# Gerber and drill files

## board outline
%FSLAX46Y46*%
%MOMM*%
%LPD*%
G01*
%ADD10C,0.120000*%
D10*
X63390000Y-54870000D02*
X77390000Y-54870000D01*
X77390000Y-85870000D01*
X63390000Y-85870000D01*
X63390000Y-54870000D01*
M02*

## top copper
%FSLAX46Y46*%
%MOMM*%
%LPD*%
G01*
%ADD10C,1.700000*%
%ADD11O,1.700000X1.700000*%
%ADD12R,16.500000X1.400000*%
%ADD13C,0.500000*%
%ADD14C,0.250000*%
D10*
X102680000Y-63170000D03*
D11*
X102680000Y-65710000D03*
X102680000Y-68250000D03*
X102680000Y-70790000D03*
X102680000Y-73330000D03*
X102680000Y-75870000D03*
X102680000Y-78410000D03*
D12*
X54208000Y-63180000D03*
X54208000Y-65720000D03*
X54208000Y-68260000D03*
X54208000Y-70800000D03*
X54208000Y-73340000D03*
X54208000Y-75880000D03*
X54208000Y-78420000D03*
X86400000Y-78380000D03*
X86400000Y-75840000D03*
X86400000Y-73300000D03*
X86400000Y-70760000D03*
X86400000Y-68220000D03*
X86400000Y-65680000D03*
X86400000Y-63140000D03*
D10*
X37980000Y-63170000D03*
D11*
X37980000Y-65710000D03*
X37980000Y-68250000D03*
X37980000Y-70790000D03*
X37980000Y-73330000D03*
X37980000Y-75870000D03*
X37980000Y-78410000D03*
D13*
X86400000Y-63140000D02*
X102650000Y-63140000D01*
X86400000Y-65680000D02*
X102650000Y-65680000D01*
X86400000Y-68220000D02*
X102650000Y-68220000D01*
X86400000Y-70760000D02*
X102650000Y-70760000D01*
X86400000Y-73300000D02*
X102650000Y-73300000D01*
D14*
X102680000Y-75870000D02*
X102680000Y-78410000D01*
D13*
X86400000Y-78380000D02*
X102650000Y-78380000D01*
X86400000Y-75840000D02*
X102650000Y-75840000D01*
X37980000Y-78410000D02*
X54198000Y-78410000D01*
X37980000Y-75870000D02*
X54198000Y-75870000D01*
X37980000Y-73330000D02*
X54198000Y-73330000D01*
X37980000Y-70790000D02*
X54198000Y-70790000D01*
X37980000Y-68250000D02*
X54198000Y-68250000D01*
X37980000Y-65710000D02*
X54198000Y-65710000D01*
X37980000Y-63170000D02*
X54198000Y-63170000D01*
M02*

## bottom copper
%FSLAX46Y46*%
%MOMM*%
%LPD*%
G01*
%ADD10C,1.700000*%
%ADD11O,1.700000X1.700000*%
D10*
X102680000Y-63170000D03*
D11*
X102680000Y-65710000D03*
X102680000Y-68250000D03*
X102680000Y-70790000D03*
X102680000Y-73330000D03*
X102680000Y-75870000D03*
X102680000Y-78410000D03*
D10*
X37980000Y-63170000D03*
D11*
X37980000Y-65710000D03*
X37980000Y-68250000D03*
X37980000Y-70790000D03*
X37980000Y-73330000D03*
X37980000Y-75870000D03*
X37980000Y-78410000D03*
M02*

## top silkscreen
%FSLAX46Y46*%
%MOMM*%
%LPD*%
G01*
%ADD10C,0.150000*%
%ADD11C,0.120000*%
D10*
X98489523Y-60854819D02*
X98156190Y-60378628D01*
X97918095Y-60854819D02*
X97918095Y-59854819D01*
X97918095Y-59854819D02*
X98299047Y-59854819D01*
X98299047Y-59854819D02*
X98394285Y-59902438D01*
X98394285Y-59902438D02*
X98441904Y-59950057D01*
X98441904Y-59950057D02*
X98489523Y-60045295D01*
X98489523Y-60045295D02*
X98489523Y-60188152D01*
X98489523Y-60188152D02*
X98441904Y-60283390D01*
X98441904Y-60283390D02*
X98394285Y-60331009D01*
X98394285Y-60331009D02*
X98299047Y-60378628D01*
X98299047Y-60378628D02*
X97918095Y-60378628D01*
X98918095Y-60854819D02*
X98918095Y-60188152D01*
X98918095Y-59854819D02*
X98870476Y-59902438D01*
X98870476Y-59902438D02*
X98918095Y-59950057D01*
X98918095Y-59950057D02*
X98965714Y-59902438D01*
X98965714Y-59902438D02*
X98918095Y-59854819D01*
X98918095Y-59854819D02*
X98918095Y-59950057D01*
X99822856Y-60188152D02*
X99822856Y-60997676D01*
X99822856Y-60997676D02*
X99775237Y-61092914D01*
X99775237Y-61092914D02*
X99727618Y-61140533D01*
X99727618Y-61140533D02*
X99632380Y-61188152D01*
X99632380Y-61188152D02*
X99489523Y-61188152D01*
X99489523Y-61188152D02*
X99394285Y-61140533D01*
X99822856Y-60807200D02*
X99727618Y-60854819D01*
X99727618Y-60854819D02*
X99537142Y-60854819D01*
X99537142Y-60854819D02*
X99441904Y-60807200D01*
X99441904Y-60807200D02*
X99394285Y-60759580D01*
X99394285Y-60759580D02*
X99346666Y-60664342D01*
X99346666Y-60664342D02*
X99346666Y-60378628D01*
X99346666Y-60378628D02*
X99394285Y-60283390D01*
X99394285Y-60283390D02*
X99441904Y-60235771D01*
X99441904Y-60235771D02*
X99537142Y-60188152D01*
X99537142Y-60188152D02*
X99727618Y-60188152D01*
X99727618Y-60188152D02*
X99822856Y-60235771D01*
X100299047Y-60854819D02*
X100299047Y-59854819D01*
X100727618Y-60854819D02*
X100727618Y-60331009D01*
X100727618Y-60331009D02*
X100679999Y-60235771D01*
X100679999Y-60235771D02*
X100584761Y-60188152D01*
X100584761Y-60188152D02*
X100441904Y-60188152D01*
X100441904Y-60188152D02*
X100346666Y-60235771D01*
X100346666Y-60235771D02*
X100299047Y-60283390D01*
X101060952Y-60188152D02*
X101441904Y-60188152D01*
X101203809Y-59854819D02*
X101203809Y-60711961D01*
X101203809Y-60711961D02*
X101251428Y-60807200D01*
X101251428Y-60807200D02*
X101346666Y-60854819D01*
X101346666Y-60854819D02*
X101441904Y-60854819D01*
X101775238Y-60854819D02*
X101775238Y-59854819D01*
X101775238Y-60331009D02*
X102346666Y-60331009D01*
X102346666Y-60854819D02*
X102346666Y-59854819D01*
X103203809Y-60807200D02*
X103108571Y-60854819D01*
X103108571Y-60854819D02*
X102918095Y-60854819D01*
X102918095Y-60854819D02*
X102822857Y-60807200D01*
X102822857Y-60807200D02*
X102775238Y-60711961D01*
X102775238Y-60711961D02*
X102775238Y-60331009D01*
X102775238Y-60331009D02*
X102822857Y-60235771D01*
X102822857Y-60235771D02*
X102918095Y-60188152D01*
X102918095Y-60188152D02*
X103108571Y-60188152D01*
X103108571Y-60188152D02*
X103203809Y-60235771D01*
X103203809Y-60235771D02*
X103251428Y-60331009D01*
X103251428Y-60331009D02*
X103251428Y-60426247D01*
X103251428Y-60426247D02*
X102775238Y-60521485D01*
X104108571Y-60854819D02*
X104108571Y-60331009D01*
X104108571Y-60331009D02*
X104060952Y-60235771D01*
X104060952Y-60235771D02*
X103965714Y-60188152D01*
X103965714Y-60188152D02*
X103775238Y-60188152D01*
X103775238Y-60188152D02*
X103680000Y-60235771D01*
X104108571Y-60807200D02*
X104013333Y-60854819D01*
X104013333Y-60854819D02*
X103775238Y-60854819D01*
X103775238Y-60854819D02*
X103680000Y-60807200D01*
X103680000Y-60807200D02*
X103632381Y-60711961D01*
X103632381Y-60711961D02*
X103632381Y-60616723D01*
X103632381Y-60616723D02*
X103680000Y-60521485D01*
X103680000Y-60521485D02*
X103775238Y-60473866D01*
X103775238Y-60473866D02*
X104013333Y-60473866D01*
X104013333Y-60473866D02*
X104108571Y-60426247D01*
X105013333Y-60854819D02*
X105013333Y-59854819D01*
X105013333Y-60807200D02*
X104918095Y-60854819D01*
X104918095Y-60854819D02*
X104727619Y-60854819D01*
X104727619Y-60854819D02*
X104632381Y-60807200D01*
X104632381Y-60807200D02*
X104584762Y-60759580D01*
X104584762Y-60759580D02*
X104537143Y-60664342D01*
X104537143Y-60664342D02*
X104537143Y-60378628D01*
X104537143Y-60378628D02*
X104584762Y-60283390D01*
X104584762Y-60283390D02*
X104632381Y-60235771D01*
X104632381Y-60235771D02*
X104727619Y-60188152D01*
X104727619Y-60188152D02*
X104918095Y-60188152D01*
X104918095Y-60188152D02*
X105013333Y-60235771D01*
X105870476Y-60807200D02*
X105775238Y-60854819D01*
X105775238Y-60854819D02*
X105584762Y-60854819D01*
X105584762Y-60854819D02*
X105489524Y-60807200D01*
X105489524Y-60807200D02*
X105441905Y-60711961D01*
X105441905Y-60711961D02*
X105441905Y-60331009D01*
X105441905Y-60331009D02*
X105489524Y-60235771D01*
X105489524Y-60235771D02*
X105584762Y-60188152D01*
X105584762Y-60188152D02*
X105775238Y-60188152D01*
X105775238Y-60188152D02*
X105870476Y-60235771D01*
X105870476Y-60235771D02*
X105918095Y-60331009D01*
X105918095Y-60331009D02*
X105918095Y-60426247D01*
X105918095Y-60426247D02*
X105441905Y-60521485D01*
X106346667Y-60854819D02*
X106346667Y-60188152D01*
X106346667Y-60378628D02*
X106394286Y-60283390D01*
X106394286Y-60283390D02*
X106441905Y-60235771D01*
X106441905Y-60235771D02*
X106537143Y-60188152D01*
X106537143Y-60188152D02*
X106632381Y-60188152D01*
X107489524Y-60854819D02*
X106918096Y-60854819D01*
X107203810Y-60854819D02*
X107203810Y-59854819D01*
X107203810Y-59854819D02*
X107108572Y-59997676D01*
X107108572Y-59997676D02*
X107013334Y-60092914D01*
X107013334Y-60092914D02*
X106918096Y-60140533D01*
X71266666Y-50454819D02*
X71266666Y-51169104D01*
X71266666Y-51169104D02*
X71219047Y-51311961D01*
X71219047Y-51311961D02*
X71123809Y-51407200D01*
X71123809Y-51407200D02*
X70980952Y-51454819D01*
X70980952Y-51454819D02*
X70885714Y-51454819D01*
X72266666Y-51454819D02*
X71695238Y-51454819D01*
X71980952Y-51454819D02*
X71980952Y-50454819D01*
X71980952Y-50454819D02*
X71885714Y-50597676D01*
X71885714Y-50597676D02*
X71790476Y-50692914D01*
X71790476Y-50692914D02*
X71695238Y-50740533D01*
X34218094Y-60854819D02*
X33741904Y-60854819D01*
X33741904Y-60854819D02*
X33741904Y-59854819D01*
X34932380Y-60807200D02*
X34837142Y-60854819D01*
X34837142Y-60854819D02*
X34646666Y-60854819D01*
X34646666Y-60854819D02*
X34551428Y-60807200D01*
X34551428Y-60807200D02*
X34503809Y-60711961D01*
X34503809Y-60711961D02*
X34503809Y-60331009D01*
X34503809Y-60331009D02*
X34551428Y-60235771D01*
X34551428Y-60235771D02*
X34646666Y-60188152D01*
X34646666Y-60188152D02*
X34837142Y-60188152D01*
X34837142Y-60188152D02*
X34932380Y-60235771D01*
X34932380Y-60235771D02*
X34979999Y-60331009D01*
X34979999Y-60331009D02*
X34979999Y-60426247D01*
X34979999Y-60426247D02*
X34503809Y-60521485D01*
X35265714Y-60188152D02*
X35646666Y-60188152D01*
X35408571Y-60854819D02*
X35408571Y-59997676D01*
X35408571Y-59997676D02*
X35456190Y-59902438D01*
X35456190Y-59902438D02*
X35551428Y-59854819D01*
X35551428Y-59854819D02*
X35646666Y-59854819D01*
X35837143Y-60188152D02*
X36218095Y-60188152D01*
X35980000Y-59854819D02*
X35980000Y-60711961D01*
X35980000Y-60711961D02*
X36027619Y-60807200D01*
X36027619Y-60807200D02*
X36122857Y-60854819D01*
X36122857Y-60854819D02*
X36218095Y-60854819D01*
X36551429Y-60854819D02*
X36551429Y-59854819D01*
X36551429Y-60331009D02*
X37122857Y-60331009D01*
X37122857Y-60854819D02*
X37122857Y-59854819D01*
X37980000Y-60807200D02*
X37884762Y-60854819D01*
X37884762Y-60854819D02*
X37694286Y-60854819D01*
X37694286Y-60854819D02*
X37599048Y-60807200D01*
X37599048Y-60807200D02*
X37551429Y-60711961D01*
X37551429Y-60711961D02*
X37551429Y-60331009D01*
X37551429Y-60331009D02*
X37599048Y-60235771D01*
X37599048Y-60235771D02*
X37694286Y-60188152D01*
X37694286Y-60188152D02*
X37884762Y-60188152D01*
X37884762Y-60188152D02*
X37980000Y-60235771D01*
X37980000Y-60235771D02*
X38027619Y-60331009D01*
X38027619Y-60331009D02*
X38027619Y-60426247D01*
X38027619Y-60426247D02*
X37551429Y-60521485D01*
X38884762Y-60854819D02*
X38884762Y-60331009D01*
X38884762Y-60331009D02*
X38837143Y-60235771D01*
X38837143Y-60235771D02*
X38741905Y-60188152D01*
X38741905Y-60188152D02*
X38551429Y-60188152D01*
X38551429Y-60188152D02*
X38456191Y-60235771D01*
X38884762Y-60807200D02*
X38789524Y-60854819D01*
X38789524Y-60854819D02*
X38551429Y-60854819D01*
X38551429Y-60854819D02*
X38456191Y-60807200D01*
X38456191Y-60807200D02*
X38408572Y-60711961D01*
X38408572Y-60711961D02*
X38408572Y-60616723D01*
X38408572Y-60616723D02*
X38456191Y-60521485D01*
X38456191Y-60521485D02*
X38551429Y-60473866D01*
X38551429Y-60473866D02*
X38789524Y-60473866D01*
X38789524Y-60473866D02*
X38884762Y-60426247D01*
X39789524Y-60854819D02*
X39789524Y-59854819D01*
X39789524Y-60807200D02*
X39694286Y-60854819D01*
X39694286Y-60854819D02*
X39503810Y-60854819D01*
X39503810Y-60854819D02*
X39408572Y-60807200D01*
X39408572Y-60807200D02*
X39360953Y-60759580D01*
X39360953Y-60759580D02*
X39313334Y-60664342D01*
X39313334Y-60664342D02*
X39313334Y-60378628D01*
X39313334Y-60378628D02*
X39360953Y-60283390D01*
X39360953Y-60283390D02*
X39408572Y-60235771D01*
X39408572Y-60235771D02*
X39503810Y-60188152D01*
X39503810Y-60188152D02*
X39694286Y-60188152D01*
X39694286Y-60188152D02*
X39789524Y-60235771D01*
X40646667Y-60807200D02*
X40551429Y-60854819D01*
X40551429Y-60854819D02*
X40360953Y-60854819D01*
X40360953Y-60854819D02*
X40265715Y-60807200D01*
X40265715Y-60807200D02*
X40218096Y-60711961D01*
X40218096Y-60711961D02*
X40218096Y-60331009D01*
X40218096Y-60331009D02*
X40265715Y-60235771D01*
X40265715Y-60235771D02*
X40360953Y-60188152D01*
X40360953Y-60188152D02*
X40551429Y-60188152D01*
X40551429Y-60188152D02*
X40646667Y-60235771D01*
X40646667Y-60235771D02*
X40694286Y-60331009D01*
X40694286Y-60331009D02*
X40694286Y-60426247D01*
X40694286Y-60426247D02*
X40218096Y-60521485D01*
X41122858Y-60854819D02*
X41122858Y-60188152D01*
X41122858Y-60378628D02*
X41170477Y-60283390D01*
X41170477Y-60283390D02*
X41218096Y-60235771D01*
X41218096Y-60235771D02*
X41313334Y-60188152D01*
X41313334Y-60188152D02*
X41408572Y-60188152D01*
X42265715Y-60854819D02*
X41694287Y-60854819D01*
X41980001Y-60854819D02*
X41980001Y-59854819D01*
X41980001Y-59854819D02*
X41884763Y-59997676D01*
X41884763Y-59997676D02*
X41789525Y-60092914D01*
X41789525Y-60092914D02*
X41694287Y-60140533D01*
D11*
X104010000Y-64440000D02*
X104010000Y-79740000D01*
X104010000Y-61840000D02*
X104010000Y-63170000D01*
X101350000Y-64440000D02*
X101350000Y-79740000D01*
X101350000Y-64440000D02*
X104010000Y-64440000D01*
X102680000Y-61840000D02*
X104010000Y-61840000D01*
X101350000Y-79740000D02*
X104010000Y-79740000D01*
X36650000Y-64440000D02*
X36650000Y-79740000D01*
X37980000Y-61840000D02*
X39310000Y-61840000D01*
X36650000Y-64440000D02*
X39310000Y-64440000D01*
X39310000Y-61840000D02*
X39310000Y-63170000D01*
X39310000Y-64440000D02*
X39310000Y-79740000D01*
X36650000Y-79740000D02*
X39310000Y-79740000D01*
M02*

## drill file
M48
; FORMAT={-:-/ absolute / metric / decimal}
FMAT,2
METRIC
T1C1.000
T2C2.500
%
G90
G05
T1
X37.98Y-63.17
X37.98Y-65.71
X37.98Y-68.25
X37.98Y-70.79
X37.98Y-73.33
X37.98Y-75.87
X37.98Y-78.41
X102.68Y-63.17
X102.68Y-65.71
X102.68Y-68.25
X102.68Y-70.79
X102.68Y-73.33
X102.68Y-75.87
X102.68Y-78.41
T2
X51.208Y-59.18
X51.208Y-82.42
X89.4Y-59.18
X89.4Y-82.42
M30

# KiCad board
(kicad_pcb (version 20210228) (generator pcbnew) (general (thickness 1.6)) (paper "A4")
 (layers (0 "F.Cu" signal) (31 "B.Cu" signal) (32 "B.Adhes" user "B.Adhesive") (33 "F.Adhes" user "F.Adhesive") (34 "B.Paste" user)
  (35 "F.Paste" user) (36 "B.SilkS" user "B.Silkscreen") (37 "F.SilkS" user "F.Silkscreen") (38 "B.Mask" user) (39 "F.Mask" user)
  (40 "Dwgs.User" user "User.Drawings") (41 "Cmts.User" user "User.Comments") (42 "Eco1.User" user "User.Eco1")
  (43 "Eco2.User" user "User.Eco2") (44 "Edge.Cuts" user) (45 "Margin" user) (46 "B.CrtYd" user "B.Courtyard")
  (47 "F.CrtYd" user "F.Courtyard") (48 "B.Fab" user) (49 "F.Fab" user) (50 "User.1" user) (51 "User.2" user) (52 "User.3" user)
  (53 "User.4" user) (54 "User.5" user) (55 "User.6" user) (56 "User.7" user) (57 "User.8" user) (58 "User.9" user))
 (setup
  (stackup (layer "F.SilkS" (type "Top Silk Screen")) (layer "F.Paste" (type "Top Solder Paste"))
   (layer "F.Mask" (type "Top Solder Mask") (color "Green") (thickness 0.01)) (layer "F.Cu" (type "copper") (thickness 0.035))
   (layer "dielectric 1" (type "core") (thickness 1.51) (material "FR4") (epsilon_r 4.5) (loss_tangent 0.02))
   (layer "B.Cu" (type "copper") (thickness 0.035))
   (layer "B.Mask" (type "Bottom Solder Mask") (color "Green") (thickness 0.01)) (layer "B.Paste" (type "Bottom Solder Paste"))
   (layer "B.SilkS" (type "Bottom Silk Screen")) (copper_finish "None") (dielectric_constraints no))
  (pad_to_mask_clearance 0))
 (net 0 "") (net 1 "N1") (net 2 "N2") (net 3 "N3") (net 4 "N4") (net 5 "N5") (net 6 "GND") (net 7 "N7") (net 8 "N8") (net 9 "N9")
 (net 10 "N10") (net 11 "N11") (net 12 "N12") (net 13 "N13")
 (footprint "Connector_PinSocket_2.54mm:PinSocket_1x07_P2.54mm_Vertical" (layer "F.Cu") (at 102.68 63.17)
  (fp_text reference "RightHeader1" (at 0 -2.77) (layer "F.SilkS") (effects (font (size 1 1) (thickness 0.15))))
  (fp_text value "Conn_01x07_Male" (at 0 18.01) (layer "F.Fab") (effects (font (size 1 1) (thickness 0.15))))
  (fp_line (start 1.33 1.27) (end 1.33 16.57) (layer "F.SilkS") (width 0.12))
  (fp_line (start 1.33 -1.33) (end 1.33 0) (layer "F.SilkS") (width 0.12))
  (fp_line (start -1.33 1.27) (end -1.33 16.57) (layer "F.SilkS") (width 0.12))
  (fp_line (start -1.33 1.27) (end 1.33 1.27) (layer "F.SilkS") (width 0.12))
  (fp_line (start 0 -1.33) (end 1.33 -1.33) (layer "F.SilkS") (width 0.12))
  (fp_line (start -1.33 16.57) (end 1.33 16.57) (layer "F.SilkS") (width 0.12))
  (pad "1" thru_hole circle (at 0 0) (locked) (size 1.7 1.7) (drill 1) (layers *.Cu *.Mask) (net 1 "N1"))
  (pad "2" thru_hole oval (at 0 2.54) (locked) (size 1.7 1.7) (drill 1) (layers *.Cu *.Mask) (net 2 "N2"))
  (pad "3" thru_hole oval (at 0 5.08) (locked) (size 1.7 1.7) (drill 1) (layers *.Cu *.Mask) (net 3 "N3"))
  (pad "4" thru_hole oval (at 0 7.62) (locked) (size 1.7 1.7) (drill 1) (layers *.Cu *.Mask) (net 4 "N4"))
  (pad "5" thru_hole oval (at 0 10.16) (locked) (size 1.7 1.7) (drill 1) (layers *.Cu *.Mask) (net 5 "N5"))
  (pad "6" thru_hole oval (at 0 12.7) (locked) (size 1.7 1.7) (drill 1) (layers *.Cu *.Mask) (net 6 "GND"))
  (pad "7" thru_hole oval (at 0 15.24) (locked) (size 1.7 1.7) (drill 1) (layers *.Cu *.Mask) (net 6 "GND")))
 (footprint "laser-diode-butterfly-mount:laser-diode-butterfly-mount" (layer "F.Cu") (at 3.48 20.87)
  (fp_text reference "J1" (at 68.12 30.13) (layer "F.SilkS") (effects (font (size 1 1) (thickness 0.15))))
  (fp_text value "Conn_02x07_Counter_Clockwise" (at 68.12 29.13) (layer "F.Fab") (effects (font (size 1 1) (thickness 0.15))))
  (fp_rect (start 59.91 34) (end 73.91 65) (layer "Edge.Cuts") (width 0.12) (fill none))
  (pad "" np_thru_hole circle (at 47.728 61.55) (size 2.5 2.5) (drill 2.5) (layers *.Mask))
  (pad "" np_thru_hole circle (at 85.92 38.31) (size 2.5 2.5) (drill 2.5) (layers *.Mask))
  (pad "" np_thru_hole circle (at 47.728 38.31) (size 2.5 2.5) (drill 2.5) (layers *.Mask))
  (pad "" np_thru_hole circle (at 85.92 61.55) (size 2.5 2.5) (drill 2.5) (layers *.Mask))
  (pad "1" smd rect (at 50.728 42.31) (locked) (size 16.5 1.4) (layers "F.Cu" "F.Paste" "F.Mask") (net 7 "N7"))
  (pad "2" smd rect (at 50.728 44.85) (locked) (size 16.5 1.4) (layers "F.Cu" "F.Paste" "F.Mask") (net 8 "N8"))
  (pad "3" smd rect (at 50.728 47.39) (locked) (size 16.5 1.4) (layers "F.Cu" "F.Paste" "F.Mask") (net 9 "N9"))
  (pad "4" smd rect (at 50.728 49.93) (locked) (size 16.5 1.4) (layers "F.Cu" "F.Paste" "F.Mask") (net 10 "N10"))
  (pad "5" smd rect (at 50.728 52.47) (locked) (size 16.5 1.4) (layers "F.Cu" "F.Paste" "F.Mask") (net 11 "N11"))
  (pad "6" smd rect (at 50.728 55.01) (locked) (size 16.5 1.4) (layers "F.Cu" "F.Paste" "F.Mask") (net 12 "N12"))
  (pad "7" smd rect (at 50.728 57.55) (locked) (size 16.5 1.4) (layers "F.Cu" "F.Paste" "F.Mask") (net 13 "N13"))
  (pad "8" smd rect (at 82.92 57.51) (locked) (size 16.5 1.4) (layers "F.Cu" "F.Paste" "F.Mask") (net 6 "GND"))
  (pad "9" smd rect (at 82.92 54.97) (locked) (size 16.5 1.4) (layers "F.Cu" "F.Paste" "F.Mask") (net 6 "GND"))
  (pad "10" smd rect (at 82.92 52.43) (locked) (size 16.5 1.4) (layers "F.Cu" "F.Paste" "F.Mask") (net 5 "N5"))
  (pad "11" smd rect (at 82.92 49.89) (locked) (size 16.5 1.4) (layers "F.Cu" "F.Paste" "F.Mask") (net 4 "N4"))
  (pad "12" smd rect (at 82.92 47.35) (locked) (size 16.5 1.4) (layers "F.Cu" "F.Paste" "F.Mask") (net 3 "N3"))
  (pad "13" smd rect (at 82.92 44.81) (locked) (size 16.5 1.4) (layers "F.Cu" "F.Paste" "F.Mask") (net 2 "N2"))
  (pad "14" smd rect (at 82.92 42.27) (locked) (size 16.5 1.4) (layers "F.Cu" "F.Paste" "F.Mask") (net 1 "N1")))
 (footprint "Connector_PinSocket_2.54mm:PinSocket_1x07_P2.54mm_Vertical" (layer "F.Cu") (at 37.98 63.17)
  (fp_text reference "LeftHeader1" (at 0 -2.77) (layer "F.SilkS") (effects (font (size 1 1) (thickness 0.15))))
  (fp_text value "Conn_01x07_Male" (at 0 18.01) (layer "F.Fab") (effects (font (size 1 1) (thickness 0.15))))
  (fp_line (start -1.33 1.27) (end -1.33 16.57) (layer "F.SilkS") (width 0.12))
  (fp_line (start 0 -1.33) (end 1.33 -1.33) (layer "F.SilkS") (width 0.12))
  (fp_line (start -1.33 1.27) (end 1.33 1.27) (layer "F.SilkS") (width 0.12))
  (fp_line (start 1.33 -1.33) (end 1.33 0) (layer "F.SilkS") (width 0.12))
  (fp_line (start 1.33 1.27) (end 1.33 16.57) (layer "F.SilkS") (width 0.12))
  (fp_line (start -1.33 16.57) (end 1.33 16.57) (layer "F.SilkS") (width 0.12))
  (pad "1" thru_hole circle (at 0 0) (locked) (size 1.7 1.7) (drill 1) (layers *.Cu *.Mask) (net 7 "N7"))
  (pad "2" thru_hole oval (at 0 2.54) (locked) (size 1.7 1.7) (drill 1) (layers *.Cu *.Mask) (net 8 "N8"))
  (pad "3" thru_hole oval (at 0 5.08) (locked) (size 1.7 1.7) (drill 1) (layers *.Cu *.Mask) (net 9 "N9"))
  (pad "4" thru_hole oval (at 0 7.62) (locked) (size 1.7 1.7) (drill 1) (layers *.Cu *.Mask) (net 10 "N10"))
  (pad "5" thru_hole oval (at 0 10.16) (locked) (size 1.7 1.7) (drill 1) (layers *.Cu *.Mask) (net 11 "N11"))
  (pad "6" thru_hole oval (at 0 12.7) (locked) (size 1.7 1.7) (drill 1) (layers *.Cu *.Mask) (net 12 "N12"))
  (pad "7" thru_hole oval (at 0 15.24) (locked) (size 1.7 1.7) (drill 1) (layers *.Cu *.Mask) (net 13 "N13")))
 (segment (start 86.4 63.14) (end 102.65 63.14) (width 0.5) (layer "F.Cu") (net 1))
 (segment (start 86.4 65.68) (end 102.65 65.68) (width 0.5) (layer "F.Cu") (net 2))
 (segment (start 86.4 68.22) (end 102.65 68.22) (width 0.5) (layer "F.Cu") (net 3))
 (segment (start 86.4 70.76) (end 102.65 70.76) (width 0.5) (layer "F.Cu") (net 4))
 (segment (start 86.4 73.3) (end 102.65 73.3) (width 0.5) (layer "F.Cu") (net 5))
 (segment (start 102.68 75.87) (end 102.68 78.41) (width 0.25) (layer "F.Cu") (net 6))
 (segment (start 86.4 78.38) (end 102.65 78.38) (width 0.5) (layer "F.Cu") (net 6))
 (segment (start 86.4 75.84) (end 102.65 75.84) (width 0.5) (layer "F.Cu") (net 6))
 (segment (start 37.98 78.41) (end 54.198 78.41) (width 0.5) (layer "F.Cu") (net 13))
 (segment (start 37.98 75.87) (end 54.198 75.87) (width 0.5) (layer "F.Cu") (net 12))
 (segment (start 37.98 73.33) (end 54.198 73.33) (width 0.5) (layer "F.Cu") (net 11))
 (segment (start 37.98 70.79) (end 54.198 70.79) (width 0.5) (layer "F.Cu") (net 10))
 (segment (start 37.98 68.25) (end 54.198 68.25) (width 0.5) (layer "F.Cu") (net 9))
 (segment (start 37.98 65.71) (end 54.198 65.71) (width 0.5) (layer "F.Cu") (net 8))
 (segment (start 37.98 63.17) (end 54.198 63.17) (width 0.5) (layer "F.Cu") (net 7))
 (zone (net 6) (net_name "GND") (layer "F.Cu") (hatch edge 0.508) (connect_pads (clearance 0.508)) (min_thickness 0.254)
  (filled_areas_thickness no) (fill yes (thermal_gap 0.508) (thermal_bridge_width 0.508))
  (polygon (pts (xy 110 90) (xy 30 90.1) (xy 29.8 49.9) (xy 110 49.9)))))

